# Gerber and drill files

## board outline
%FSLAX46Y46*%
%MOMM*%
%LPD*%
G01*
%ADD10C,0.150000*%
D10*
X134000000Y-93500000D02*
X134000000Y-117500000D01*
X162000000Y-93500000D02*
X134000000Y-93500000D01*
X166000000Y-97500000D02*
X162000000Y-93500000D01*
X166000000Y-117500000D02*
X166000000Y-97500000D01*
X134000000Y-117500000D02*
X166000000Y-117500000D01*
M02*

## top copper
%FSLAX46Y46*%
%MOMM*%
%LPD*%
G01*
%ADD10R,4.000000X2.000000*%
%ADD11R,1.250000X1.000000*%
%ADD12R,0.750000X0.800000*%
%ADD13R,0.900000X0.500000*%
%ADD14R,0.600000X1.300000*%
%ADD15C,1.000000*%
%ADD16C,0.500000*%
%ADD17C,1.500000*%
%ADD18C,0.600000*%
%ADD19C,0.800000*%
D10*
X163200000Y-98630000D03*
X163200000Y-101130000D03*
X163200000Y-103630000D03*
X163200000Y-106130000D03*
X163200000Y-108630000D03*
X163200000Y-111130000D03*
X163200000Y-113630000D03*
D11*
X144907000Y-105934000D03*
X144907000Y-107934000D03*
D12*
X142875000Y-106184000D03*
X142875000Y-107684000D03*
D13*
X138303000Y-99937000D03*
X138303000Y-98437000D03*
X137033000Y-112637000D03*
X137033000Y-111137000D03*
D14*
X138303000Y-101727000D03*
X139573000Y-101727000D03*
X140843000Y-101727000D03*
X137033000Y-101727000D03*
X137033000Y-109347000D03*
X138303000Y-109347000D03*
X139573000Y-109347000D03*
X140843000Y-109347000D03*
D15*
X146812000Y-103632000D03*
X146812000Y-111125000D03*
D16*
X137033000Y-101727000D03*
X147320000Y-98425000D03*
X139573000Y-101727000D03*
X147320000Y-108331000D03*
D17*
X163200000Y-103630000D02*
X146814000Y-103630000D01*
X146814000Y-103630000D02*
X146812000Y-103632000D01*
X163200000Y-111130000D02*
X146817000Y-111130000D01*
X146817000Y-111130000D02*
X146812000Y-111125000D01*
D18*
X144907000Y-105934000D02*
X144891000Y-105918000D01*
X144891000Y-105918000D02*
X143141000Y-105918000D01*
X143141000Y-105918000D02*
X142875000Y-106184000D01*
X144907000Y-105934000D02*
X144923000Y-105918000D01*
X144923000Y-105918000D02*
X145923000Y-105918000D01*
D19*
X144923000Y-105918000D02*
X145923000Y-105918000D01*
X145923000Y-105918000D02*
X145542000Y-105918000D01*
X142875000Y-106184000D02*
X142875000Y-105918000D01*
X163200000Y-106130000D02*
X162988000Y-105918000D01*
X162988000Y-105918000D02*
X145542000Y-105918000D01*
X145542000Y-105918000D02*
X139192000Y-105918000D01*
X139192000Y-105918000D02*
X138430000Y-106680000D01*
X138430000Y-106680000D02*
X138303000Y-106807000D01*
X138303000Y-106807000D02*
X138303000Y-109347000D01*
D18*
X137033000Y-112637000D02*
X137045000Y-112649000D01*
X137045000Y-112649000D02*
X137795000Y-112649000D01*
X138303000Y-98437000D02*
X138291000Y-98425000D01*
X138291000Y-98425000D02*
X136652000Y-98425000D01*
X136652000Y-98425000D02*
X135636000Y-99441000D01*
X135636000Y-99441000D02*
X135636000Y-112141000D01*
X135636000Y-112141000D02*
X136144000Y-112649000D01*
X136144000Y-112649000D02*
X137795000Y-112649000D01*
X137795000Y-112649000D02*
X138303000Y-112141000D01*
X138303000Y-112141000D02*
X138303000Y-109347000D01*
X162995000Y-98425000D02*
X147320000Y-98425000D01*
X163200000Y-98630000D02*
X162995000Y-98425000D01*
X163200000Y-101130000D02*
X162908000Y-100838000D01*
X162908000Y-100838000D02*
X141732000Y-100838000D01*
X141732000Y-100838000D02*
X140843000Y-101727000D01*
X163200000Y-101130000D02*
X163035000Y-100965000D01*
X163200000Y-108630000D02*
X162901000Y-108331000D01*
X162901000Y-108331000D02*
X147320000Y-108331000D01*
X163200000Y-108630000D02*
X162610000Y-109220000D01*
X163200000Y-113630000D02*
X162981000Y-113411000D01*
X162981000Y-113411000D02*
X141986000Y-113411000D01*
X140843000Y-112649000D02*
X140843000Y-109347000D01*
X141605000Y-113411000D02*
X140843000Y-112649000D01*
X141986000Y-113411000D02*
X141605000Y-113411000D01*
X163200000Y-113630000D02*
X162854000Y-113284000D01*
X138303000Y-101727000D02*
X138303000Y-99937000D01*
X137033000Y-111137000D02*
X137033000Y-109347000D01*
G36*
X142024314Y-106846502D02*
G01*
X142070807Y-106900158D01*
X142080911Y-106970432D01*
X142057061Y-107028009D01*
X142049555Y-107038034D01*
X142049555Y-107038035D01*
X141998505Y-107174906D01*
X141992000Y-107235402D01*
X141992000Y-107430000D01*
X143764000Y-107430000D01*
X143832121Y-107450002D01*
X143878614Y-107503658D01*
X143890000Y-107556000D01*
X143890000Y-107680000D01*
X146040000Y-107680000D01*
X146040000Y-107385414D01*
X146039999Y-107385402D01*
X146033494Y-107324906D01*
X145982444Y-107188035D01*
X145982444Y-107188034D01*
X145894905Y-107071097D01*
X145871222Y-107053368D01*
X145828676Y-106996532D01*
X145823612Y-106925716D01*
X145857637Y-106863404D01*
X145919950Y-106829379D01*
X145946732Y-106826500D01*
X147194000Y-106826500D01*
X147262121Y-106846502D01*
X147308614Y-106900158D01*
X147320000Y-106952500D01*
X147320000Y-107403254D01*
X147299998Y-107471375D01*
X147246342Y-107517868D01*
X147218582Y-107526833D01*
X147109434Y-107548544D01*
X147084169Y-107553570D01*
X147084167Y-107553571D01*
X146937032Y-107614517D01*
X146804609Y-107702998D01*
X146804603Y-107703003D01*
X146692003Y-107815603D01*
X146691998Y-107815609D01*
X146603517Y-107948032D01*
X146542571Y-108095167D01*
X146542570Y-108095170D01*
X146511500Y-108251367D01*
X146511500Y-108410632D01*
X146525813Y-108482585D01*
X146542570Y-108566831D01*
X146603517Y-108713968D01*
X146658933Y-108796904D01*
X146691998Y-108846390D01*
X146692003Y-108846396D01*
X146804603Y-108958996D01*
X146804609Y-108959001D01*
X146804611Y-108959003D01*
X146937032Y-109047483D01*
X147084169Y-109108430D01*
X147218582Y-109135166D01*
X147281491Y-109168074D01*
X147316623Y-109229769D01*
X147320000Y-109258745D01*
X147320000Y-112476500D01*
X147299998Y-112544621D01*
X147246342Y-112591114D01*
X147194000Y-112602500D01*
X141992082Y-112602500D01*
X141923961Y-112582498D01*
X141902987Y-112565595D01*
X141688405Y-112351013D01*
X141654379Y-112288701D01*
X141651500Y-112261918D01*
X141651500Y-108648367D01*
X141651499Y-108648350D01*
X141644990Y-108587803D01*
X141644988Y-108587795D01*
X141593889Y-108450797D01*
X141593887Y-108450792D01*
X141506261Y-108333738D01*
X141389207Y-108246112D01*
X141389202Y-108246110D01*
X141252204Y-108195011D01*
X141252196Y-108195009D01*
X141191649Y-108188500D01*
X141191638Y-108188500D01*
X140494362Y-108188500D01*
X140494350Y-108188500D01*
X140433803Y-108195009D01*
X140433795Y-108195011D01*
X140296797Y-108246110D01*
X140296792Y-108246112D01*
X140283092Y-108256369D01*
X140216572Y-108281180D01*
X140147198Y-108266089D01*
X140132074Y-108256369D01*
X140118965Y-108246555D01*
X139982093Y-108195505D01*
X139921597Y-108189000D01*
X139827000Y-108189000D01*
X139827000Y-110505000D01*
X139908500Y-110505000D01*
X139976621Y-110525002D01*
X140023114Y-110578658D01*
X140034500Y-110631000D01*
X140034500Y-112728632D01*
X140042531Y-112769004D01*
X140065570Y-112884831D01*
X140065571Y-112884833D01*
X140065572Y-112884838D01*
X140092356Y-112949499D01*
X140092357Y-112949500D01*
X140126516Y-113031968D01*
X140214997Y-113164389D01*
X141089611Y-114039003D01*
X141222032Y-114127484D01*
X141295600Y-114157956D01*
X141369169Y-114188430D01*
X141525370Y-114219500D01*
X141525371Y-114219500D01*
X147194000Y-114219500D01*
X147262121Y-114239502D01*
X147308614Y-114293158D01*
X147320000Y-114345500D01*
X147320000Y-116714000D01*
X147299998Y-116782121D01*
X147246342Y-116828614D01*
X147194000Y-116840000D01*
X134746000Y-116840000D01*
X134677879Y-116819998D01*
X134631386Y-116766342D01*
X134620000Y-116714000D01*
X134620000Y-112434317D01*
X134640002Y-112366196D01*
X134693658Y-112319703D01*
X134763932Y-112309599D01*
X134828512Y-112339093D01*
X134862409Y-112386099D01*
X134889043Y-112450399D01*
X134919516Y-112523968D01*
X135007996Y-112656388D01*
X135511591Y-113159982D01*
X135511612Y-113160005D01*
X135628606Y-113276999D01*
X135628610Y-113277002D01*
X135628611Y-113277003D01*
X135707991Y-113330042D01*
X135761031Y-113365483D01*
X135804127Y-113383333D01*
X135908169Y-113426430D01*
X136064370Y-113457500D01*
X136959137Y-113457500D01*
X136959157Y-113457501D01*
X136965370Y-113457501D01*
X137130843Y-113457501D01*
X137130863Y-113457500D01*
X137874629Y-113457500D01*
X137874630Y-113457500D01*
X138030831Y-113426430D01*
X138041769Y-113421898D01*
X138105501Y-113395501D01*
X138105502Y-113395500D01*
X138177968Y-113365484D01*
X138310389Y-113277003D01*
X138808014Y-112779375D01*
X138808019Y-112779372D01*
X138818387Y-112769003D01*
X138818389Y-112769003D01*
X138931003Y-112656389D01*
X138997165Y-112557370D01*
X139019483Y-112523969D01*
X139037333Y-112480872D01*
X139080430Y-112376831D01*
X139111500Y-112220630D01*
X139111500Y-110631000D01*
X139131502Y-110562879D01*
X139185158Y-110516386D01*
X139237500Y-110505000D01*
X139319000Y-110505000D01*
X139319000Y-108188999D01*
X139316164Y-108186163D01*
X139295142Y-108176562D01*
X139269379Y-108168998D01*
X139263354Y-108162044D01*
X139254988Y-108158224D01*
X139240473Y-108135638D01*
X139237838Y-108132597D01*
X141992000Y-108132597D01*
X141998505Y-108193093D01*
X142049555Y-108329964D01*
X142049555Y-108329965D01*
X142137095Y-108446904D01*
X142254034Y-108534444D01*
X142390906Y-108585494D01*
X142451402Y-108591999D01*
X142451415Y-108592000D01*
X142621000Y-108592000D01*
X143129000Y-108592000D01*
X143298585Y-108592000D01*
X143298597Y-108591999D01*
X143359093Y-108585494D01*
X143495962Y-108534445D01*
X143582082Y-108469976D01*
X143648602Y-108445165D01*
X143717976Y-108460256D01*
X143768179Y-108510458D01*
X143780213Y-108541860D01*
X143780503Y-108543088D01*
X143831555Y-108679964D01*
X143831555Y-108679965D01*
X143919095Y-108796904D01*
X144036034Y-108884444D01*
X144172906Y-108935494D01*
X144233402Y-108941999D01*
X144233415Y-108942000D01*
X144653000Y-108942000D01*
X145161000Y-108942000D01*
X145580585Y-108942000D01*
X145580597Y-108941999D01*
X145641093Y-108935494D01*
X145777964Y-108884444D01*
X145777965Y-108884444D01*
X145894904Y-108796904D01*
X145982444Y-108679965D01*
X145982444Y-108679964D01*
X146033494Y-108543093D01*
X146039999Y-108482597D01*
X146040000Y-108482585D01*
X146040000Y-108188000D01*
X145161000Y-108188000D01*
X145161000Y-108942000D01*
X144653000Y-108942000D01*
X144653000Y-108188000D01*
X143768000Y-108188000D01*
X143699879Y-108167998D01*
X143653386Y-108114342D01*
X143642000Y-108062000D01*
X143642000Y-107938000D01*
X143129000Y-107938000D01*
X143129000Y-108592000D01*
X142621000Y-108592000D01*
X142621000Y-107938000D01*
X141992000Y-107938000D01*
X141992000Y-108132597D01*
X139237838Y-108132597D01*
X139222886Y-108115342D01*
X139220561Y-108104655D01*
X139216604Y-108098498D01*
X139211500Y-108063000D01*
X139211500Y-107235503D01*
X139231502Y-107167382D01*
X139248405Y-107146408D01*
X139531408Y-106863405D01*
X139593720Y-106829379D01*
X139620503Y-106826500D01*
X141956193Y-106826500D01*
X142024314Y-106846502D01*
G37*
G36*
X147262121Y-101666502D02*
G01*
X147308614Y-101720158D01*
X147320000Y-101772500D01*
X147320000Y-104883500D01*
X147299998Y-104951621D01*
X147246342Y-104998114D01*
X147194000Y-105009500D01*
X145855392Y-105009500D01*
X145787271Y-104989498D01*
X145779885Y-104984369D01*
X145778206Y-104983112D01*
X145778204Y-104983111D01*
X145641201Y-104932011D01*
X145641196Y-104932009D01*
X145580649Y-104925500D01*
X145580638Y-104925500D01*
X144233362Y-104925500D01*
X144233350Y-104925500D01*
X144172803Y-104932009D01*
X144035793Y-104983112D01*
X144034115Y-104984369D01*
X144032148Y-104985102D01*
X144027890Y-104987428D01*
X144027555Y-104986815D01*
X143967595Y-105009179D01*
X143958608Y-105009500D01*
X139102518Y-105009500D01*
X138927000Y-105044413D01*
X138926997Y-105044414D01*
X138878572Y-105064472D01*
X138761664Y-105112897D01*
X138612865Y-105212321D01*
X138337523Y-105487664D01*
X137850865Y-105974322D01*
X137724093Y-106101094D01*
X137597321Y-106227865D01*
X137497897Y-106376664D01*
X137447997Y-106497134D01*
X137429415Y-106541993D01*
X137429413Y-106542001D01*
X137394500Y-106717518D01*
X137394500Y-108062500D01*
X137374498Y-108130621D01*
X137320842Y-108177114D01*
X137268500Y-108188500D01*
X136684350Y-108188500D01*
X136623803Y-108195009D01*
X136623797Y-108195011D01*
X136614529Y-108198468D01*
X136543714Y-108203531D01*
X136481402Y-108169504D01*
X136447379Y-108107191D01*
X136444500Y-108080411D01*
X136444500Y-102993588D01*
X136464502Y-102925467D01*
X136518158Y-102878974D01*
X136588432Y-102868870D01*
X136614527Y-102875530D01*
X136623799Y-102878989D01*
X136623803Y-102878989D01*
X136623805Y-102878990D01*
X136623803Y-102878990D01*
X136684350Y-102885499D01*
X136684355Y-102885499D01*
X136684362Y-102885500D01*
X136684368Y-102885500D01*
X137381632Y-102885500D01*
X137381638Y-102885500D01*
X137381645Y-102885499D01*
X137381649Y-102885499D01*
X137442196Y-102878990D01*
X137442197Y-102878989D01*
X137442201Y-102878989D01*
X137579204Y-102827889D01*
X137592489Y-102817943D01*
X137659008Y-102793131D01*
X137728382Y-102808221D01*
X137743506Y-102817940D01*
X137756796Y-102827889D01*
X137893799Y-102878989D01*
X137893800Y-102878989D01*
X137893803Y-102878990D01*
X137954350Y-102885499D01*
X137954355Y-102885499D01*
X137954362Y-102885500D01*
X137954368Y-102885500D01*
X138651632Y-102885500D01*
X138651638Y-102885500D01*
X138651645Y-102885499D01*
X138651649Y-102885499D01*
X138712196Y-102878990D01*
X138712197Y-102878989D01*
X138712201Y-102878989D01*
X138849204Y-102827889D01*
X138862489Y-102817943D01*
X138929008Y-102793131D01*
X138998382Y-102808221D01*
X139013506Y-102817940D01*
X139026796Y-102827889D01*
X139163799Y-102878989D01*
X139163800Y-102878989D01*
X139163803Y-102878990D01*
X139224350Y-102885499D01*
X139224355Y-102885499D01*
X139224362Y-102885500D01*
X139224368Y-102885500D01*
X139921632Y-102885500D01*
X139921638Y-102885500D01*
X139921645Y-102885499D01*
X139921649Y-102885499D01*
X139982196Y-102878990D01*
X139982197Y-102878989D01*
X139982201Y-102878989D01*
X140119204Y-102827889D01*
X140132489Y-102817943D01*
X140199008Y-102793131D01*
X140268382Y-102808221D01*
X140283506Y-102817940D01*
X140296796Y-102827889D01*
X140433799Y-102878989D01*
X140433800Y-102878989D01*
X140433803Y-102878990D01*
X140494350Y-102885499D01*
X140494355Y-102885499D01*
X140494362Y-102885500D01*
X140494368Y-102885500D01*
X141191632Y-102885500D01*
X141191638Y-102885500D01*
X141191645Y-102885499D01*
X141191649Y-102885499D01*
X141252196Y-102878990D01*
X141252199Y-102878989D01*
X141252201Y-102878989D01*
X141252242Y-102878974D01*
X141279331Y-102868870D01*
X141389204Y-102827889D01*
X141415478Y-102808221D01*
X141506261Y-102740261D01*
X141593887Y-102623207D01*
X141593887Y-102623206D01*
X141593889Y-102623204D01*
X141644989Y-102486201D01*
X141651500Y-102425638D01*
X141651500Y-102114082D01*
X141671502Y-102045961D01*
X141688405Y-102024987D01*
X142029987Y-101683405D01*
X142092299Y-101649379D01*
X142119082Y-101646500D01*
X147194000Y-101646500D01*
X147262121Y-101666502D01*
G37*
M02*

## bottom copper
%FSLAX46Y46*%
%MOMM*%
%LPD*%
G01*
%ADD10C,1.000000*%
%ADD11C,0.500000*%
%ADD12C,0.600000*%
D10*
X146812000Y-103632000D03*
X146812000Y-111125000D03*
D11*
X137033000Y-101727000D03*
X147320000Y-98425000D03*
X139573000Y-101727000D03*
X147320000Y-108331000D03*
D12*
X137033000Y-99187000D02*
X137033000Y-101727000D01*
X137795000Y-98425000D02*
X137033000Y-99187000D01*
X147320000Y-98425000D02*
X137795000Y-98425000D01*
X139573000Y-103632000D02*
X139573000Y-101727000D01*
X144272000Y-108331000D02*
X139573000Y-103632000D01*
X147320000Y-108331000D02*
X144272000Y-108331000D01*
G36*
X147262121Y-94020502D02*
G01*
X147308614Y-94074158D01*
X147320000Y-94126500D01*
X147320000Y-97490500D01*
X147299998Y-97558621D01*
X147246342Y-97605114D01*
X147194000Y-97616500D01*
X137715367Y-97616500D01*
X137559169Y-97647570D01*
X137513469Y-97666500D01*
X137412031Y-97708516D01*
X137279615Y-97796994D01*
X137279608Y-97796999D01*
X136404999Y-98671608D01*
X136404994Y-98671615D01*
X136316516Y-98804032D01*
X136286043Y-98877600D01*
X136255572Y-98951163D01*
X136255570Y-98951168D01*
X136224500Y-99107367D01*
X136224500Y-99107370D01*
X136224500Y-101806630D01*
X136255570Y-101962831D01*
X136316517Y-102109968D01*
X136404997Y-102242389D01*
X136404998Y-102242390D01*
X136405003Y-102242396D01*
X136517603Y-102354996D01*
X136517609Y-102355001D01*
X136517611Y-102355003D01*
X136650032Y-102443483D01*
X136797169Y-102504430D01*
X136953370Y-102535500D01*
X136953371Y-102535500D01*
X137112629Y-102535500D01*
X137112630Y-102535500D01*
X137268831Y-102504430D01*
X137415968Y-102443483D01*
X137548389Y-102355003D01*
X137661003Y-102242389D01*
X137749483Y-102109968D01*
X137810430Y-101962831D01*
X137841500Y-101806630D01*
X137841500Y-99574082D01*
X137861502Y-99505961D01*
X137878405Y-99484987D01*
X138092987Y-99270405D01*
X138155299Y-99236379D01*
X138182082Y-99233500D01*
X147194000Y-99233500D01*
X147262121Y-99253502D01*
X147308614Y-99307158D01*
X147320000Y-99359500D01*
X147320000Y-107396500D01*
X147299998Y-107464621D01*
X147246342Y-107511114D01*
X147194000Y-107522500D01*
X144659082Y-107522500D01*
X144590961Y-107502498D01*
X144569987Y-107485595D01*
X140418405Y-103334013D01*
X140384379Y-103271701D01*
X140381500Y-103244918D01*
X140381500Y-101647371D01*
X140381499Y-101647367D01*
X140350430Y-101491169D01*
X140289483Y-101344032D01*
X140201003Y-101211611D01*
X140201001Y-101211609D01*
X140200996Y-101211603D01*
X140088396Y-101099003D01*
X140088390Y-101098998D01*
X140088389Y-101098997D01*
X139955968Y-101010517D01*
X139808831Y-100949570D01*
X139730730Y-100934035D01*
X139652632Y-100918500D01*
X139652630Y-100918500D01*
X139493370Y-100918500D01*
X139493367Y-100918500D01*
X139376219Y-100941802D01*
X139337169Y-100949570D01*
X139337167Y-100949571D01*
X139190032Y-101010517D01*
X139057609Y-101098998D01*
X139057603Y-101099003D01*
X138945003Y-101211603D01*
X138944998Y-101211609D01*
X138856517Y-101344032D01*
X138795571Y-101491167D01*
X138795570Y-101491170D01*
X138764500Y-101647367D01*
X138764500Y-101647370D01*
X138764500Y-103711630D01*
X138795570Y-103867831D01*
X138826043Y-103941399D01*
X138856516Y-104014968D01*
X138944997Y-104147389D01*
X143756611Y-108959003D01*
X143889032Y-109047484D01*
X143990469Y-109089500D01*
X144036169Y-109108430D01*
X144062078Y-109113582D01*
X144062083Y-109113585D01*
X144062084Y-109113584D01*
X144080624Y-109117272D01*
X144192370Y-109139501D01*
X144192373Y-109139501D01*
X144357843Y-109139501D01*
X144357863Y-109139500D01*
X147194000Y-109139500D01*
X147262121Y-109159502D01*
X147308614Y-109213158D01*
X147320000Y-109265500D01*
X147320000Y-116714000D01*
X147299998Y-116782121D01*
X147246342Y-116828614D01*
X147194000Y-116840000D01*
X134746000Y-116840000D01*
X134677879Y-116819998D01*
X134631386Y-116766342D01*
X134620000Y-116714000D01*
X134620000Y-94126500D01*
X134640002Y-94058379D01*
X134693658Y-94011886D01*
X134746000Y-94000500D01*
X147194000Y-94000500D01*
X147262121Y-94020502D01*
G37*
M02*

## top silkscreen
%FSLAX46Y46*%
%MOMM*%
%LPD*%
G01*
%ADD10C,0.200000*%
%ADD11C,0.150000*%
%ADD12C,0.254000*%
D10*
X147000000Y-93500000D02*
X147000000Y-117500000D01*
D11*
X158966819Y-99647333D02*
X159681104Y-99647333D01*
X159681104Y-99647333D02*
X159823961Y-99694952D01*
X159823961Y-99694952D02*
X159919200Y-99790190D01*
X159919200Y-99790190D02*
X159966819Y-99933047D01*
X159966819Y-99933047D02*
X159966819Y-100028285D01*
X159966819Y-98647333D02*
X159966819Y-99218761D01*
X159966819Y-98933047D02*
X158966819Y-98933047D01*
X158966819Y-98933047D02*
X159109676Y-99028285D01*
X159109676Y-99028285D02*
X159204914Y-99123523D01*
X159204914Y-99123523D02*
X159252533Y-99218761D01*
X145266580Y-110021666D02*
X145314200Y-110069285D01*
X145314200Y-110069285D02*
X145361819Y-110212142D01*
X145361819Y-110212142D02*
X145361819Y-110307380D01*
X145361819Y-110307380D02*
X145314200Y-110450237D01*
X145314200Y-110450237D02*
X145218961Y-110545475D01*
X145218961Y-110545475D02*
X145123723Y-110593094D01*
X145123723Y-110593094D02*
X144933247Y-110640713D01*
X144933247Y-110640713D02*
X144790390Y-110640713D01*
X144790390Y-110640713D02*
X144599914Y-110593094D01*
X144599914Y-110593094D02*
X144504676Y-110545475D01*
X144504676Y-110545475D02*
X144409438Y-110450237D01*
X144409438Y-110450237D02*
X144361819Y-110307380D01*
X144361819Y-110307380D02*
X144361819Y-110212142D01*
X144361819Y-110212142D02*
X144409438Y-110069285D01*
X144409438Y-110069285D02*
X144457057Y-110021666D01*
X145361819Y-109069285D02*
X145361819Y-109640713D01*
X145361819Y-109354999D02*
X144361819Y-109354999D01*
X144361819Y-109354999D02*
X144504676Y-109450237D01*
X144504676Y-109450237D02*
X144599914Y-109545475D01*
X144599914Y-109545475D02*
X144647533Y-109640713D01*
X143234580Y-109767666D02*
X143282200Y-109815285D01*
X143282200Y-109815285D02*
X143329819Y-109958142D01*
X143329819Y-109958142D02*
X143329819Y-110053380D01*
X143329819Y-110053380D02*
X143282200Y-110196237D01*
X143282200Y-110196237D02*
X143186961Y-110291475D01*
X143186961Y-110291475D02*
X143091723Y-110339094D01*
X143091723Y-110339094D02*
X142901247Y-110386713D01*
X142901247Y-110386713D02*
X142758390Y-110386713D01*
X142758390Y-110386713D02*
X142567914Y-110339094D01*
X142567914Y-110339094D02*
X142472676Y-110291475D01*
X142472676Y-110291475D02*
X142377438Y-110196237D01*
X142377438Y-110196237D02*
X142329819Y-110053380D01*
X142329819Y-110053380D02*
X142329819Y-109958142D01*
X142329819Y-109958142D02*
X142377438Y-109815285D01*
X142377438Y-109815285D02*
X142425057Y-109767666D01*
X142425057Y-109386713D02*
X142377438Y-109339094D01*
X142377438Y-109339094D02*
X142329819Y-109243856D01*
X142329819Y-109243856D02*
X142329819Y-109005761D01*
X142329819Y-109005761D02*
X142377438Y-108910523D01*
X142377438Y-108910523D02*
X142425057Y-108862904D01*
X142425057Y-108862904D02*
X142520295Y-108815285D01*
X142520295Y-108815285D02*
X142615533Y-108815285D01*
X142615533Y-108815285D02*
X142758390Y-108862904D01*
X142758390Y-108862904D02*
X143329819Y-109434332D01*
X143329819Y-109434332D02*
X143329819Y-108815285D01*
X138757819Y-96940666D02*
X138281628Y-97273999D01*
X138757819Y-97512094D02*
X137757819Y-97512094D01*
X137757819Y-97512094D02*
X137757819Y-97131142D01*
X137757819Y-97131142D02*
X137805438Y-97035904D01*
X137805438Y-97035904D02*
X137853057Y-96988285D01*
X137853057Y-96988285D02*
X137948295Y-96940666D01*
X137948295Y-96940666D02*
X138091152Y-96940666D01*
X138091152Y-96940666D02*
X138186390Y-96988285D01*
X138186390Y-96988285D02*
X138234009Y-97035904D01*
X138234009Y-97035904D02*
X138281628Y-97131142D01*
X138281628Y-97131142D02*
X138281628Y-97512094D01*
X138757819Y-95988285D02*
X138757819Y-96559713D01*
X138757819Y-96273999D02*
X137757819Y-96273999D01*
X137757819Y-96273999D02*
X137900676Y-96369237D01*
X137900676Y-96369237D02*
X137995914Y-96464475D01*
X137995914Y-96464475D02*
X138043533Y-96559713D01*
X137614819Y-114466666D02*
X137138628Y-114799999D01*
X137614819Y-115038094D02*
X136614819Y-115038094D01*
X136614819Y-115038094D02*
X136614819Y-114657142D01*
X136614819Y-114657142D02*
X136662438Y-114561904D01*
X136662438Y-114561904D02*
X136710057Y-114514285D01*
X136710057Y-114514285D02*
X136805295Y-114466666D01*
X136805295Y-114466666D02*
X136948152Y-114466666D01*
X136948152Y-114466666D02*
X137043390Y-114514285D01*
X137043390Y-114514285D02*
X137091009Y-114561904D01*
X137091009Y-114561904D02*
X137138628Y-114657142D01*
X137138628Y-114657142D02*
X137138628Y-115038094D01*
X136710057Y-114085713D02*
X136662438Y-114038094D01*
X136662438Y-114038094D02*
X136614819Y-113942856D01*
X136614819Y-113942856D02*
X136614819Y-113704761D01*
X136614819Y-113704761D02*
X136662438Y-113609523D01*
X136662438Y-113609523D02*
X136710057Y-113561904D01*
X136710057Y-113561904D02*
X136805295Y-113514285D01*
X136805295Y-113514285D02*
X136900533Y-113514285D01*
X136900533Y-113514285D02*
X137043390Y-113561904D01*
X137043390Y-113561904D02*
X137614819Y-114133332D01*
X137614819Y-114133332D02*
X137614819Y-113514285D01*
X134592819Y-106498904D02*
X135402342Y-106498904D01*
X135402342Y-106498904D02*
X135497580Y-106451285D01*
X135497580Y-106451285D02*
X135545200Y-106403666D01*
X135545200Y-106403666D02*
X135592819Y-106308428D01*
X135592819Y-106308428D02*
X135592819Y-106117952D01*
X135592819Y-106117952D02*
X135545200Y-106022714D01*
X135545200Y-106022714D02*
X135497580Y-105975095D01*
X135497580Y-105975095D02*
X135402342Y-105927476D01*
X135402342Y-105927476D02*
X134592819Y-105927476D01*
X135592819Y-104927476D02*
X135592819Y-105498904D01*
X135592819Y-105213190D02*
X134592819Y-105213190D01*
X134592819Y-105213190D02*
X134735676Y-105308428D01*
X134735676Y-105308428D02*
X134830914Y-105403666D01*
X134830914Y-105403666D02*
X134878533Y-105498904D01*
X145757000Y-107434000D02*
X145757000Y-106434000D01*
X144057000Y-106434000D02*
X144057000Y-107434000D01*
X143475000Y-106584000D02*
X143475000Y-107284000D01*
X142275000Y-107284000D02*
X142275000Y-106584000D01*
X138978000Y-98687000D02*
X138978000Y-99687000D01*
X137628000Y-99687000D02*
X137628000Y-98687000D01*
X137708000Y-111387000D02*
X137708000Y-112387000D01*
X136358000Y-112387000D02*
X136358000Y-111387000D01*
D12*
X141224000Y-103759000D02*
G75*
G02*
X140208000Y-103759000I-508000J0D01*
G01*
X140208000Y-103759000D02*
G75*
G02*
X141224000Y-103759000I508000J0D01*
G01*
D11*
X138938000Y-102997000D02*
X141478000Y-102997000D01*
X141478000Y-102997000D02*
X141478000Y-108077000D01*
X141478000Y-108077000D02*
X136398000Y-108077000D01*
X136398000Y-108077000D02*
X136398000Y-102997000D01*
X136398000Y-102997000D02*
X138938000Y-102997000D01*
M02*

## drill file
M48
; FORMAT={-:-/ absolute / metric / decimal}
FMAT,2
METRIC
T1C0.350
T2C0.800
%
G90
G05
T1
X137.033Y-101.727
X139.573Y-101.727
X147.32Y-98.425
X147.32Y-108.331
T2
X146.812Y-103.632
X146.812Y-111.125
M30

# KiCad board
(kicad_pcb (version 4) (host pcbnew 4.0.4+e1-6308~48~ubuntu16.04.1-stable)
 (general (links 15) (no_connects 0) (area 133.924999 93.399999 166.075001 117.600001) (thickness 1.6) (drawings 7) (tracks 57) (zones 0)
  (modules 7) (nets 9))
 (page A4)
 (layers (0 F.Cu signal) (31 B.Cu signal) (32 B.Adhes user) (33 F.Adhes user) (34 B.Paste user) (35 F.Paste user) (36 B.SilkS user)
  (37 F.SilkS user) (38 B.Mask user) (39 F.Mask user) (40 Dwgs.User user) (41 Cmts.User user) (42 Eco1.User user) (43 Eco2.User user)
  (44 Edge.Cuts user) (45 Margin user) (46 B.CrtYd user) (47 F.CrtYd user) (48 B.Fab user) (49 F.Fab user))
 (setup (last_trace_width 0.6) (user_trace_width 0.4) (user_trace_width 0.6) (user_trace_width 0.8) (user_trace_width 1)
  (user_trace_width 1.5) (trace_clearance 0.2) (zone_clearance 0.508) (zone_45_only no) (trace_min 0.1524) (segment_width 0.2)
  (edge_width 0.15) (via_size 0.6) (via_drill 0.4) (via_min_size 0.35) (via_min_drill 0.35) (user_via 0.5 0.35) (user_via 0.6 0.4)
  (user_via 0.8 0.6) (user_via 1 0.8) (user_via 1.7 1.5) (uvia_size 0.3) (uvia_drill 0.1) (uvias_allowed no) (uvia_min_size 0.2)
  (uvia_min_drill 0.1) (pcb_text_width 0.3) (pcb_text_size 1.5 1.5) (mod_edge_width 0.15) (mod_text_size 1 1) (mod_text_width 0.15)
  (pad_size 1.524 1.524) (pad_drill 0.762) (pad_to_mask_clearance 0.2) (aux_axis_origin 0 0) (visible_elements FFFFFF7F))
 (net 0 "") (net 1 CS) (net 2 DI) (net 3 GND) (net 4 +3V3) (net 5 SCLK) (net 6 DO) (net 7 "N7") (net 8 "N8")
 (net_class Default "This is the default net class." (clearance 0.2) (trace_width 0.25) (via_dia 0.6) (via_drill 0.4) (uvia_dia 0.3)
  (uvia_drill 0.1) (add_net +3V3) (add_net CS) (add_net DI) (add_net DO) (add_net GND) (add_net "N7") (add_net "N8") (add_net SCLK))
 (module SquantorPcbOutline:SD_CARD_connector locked (layer F.Cu) (at 163.2 106.13)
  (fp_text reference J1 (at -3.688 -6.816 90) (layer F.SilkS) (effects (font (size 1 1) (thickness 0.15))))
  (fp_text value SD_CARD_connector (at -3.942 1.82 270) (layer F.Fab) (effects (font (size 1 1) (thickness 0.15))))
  (pad 1 smd rect (at 0 -7.5 90) (size 2 4) (layers F.Cu F.Paste F.Mask) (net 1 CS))
  (pad 2 smd rect (at 0 -5 90) (size 2 4) (layers F.Cu F.Paste F.Mask) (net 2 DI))
  (pad 3 smd rect (at 0 -2.5 90) (size 2 4) (layers F.Cu F.Paste F.Mask) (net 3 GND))
  (pad 4 smd rect (at 0 0 90) (size 2 4) (layers F.Cu F.Paste F.Mask) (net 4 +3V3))
  (pad 5 smd rect (at 0 2.5 90) (size 2 4) (layers F.Cu F.Paste F.Mask) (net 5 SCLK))
  (pad 6 smd rect (at 0 5 90) (size 2 4) (layers F.Cu F.Paste F.Mask) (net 3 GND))
  (pad 7 smd rect (at 0 7.5 90) (size 2 4) (layers F.Cu F.Paste F.Mask) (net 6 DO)))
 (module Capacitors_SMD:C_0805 (layer F.Cu) (at 144.907 106.934 270)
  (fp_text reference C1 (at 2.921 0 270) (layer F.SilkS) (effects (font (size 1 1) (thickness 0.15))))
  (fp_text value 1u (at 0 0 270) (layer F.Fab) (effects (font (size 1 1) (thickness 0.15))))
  (fp_line (start 0.5 -0.85) (end -0.5 -0.85) (layer F.SilkS) (width 0.15))
  (fp_line (start -0.5 0.85) (end 0.5 0.85) (layer F.SilkS) (width 0.15))
  (pad 1 smd rect (at -1 0 270) (size 1 1.25) (layers F.Cu F.Paste F.Mask) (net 4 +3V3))
  (pad 2 smd rect (at 1 0 270) (size 1 1.25) (layers F.Cu F.Paste F.Mask) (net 3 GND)))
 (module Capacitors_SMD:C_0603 (layer F.Cu) (at 142.875 106.934 270)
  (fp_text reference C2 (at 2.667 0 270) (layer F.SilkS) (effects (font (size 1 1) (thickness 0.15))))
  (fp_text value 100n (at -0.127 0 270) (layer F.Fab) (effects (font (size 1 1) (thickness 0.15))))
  (fp_line (start -0.35 -0.6) (end 0.35 -0.6) (layer F.SilkS) (width 0.15))
  (fp_line (start 0.35 0.6) (end -0.35 0.6) (layer F.SilkS) (width 0.15))
  (pad 1 smd rect (at -0.75 0 270) (size 0.8 0.75) (layers F.Cu F.Paste F.Mask) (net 4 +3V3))
  (pad 2 smd rect (at 0.75 0 270) (size 0.8 0.75) (layers F.Cu F.Paste F.Mask) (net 3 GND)))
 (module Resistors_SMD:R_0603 (layer F.Cu) (at 138.303 99.187 90)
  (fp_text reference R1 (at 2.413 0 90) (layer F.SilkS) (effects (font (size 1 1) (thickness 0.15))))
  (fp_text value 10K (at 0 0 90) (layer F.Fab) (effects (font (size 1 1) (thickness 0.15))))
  (fp_line (start 0.5 0.675) (end -0.5 0.675) (layer F.SilkS) (width 0.15))
  (fp_line (start -0.5 -0.675) (end 0.5 -0.675) (layer F.SilkS) (width 0.15))
  (pad 1 smd rect (at -0.75 0 90) (size 0.5 0.9) (layers F.Cu F.Paste F.Mask) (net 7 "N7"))
  (pad 2 smd rect (at 0.75 0 90) (size 0.5 0.9) (layers F.Cu F.Paste F.Mask) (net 4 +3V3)))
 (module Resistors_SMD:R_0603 (layer F.Cu) (at 137.033 111.887 90)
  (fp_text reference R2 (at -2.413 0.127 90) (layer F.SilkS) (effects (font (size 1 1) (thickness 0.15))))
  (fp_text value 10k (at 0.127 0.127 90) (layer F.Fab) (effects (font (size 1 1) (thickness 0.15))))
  (fp_line (start 0.5 0.675) (end -0.5 0.675) (layer F.SilkS) (width 0.15))
  (fp_line (start -0.5 -0.675) (end 0.5 -0.675) (layer F.SilkS) (width 0.15))
  (pad 1 smd rect (at -0.75 0 90) (size 0.5 0.9) (layers F.Cu F.Paste F.Mask) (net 4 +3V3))
  (pad 2 smd rect (at 0.75 0 90) (size 0.5 0.9) (layers F.Cu F.Paste F.Mask) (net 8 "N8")))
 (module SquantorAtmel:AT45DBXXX (layer F.Cu) (at 138.938 105.537 270)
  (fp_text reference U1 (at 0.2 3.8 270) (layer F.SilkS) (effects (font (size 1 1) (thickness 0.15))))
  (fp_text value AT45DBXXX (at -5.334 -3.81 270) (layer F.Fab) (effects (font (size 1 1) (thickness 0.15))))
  (fp_circle (center -1.778 -1.778) (end -1.27 -1.778) (layer F.SilkS) (width 0.254))
  (fp_line (start -2.54 0) (end -2.54 -2.54) (layer F.SilkS) (width 0.15))
  (fp_line (start -2.54 -2.54) (end 2.54 -2.54) (layer F.SilkS) (width 0.15))
  (fp_line (start 2.54 -2.54) (end 2.54 2.54) (layer F.SilkS) (width 0.15))
  (fp_line (start 2.54 2.54) (end -2.54 2.54) (layer F.SilkS) (width 0.15))
  (fp_line (start -2.54 2.54) (end -2.54 0) (layer F.SilkS) (width 0.15))
  (pad 3 smd rect (at -3.81 0.635 270) (size 1.3 0.6) (layers F.Cu F.Paste F.Mask) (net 7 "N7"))
  (pad 2 smd rect (at -3.81 -0.635 270) (size 1.3 0.6) (layers F.Cu F.Paste F.Mask) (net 5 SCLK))
  (pad 1 smd rect (at -3.81 -1.905 270) (size 1.3 0.6) (layers F.Cu F.Paste F.Mask) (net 2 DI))
  (pad 4 smd rect (at -3.81 1.905 270) (size 1.3 0.6) (layers F.Cu F.Paste F.Mask) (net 1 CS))
  (pad 5 smd rect (at 3.81 1.905 270) (size 1.3 0.6) (layers F.Cu F.Paste F.Mask) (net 8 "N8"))
  (pad 6 smd rect (at 3.81 0.635 270) (size 1.3 0.6) (layers F.Cu F.Paste F.Mask) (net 4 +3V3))
  (pad 7 smd rect (at 3.81 -0.635 270) (size 1.3 0.6) (layers F.Cu F.Paste F.Mask) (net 3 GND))
  (pad 8 smd rect (at 3.81 -1.905 270) (size 1.3 0.6) (layers F.Cu F.Paste F.Mask) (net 6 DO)))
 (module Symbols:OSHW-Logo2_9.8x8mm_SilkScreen (layer B.Cu) (at 141.859 105.156 270)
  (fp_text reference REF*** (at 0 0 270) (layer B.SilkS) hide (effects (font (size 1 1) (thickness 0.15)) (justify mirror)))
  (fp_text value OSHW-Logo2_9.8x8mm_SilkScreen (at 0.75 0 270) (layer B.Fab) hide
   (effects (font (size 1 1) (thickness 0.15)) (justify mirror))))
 (gr_line (start 147 93.5) (end 147 117.5) (angle 90) (layer F.SilkS) (width 0.2))
 (gr_line (start 134 93.5) (end 134 117.5) (angle 90) (layer Edge.Cuts) (width 0.15))
 (gr_line (start 162 93.5) (end 134 93.5) (angle 90) (layer Edge.Cuts) (width 0.15))
 (gr_line (start 166 97.5) (end 162 93.5) (angle 90) (layer Edge.Cuts) (width 0.15))
 (gr_line (start 166 117.5) (end 166 97.5) (angle 90) (layer Edge.Cuts) (width 0.15))
 (gr_line (start 134 117.5) (end 166 117.5) (angle 90) (layer Edge.Cuts) (width 0.15))
 (segment (start 163.2 103.63) (end 146.814 103.63) (width 1.5) (layer F.Cu) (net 3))
 (via (at 146.812 103.632) (size 1) (drill 0.8) (layers F.Cu B.Cu) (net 3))
 (segment (start 146.814 103.63) (end 146.812 103.632) (width 1.5) (layer F.Cu) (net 3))
 (segment (start 163.2 111.13) (end 146.817 111.13) (width 1.5) (layer F.Cu) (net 3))
 (segment (start 146.817 111.13) (end 146.812 111.125) (width 1.5) (layer F.Cu) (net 3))
 (via (at 146.812 111.125) (size 1) (drill 0.8) (layers F.Cu B.Cu) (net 3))
 (segment (start 144.907 105.934) (end 144.891 105.918) (width 0.6) (layer F.Cu) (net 4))
 (segment (start 144.891 105.918) (end 143.141 105.918) (width 0.6) (layer F.Cu) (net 4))
 (segment (start 143.141 105.918) (end 142.875 106.184) (width 0.6) (layer F.Cu) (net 4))
 (segment (start 144.907 105.934) (end 144.923 105.918) (width 0.6) (layer F.Cu) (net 4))
 (segment (start 144.923 105.918) (end 145.923 105.918) (width 0.6) (layer F.Cu) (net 4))
 (segment (start 144.923 105.918) (end 145.923 105.918) (width 0.8) (layer F.Cu) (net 4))
 (segment (start 145.923 105.918) (end 145.542 105.918) (width 0.8) (layer F.Cu) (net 4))
 (segment (start 142.875 106.184) (end 142.875 105.918) (width 0.8) (layer F.Cu) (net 4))
 (segment (start 163.2 106.13) (end 162.988 105.918) (width 0.8) (layer F.Cu) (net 4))
 (segment (start 162.988 105.918) (end 145.542 105.918) (width 0.8) (layer F.Cu) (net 4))
 (segment (start 145.542 105.918) (end 139.192 105.918) (width 0.8) (layer F.Cu) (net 4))
 (segment (start 139.192 105.918) (end 138.43 106.68) (width 0.8) (layer F.Cu) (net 4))
 (segment (start 138.43 106.68) (end 138.303 106.807) (width 0.8) (layer F.Cu) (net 4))
 (segment (start 138.303 106.807) (end 138.303 109.347) (width 0.8) (layer F.Cu) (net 4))
 (segment (start 137.033 112.637) (end 137.045 112.649) (width 0.6) (layer F.Cu) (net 4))
 (segment (start 137.045 112.649) (end 137.795 112.649) (width 0.6) (layer F.Cu) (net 4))
 (segment (start 138.303 98.437) (end 138.291 98.425) (width 0.6) (layer F.Cu) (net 4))
 (segment (start 138.291 98.425) (end 136.652 98.425) (width 0.6) (layer F.Cu) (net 4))
 (segment (start 136.652 98.425) (end 135.636 99.441) (width 0.6) (layer F.Cu) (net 4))
 (segment (start 135.636 99.441) (end 135.636 112.141) (width 0.6) (layer F.Cu) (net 4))
 (segment (start 135.636 112.141) (end 136.144 112.649) (width 0.6) (layer F.Cu) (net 4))
 (segment (start 136.144 112.649) (end 137.795 112.649) (width 0.6) (layer F.Cu) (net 4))
 (segment (start 137.795 112.649) (end 138.303 112.141) (width 0.6) (layer F.Cu) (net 4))
 (segment (start 138.303 112.141) (end 138.303 109.347) (width 0.6) (layer F.Cu) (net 4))
 (via (at 137.033 101.727) (size 0.5) (drill 0.35) (layers F.Cu B.Cu) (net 1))
 (segment (start 137.033 99.187) (end 137.033 101.727) (width 0.6) (layer B.Cu) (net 1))
 (segment (start 137.795 98.425) (end 137.033 99.187) (width 0.6) (layer B.Cu) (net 1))
 (segment (start 147.32 98.425) (end 137.795 98.425) (width 0.6) (layer B.Cu) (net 1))
 (via (at 147.32 98.425) (size 0.5) (drill 0.35) (layers F.Cu B.Cu) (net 1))
 (segment (start 162.995 98.425) (end 147.32 98.425) (width 0.6) (layer F.Cu) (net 1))
 (segment (start 163.2 98.63) (end 162.995 98.425) (width 0.6) (layer F.Cu) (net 1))
 (segment (start 163.2 101.13) (end 162.908 100.838) (width 0.6) (layer F.Cu) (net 2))
 (segment (start 162.908 100.838) (end 141.732 100.838) (width 0.6) (layer F.Cu) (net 2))
 (segment (start 141.732 100.838) (end 140.843 101.727) (width 0.6) (layer F.Cu) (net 2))
 (segment (start 163.2 101.13) (end 163.035 100.965) (width 0.6) (layer F.Cu) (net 2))
 (segment (start 163.2 108.63) (end 162.901 108.331) (width 0.6) (layer F.Cu) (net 5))
 (segment (start 162.901 108.331) (end 147.32 108.331) (width 0.6) (layer F.Cu) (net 5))
 (via (at 139.573 101.727) (size 0.5) (drill 0.35) (layers F.Cu B.Cu) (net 5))
 (segment (start 139.573 103.632) (end 139.573 101.727) (width 0.6) (layer B.Cu) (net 5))
 (segment (start 144.272 108.331) (end 139.573 103.632) (width 0.6) (layer B.Cu) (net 5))
 (segment (start 147.32 108.331) (end 144.272 108.331) (width 0.6) (layer B.Cu) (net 5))
 (via (at 147.32 108.331) (size 0.5) (drill 0.35) (layers F.Cu B.Cu) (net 5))
 (segment (start 163.2 108.63) (end 162.61 109.22) (width 0.6) (layer F.Cu) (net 5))
 (segment (start 163.2 113.63) (end 162.981 113.411) (width 0.6) (layer F.Cu) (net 6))
 (segment (start 162.981 113.411) (end 141.986 113.411) (width 0.6) (layer F.Cu) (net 6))
 (segment (start 140.843 112.649) (end 140.843 109.347) (width 0.6) (layer F.Cu) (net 6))
 (segment (start 141.605 113.411) (end 140.843 112.649) (width 0.6) (layer F.Cu) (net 6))
 (segment (start 141.986 113.411) (end 141.605 113.411) (width 0.6) (layer F.Cu) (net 6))
 (segment (start 163.2 113.63) (end 162.854 113.284) (width 0.6) (layer F.Cu) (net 6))
 (segment (start 138.303 101.727) (end 138.303 99.937) (width 0.6) (layer F.Cu) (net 7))
 (segment (start 137.033 111.137) (end 137.033 109.347) (width 0.6) (layer F.Cu) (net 8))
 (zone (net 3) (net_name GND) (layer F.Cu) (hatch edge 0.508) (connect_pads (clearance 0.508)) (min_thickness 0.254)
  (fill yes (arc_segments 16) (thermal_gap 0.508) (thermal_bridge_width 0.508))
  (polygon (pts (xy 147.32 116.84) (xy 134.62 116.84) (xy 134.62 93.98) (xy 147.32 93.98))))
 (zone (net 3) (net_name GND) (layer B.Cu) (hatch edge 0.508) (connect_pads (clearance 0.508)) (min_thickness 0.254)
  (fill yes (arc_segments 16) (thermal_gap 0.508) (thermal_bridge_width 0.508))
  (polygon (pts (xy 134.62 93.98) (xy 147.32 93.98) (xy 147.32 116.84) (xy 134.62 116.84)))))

